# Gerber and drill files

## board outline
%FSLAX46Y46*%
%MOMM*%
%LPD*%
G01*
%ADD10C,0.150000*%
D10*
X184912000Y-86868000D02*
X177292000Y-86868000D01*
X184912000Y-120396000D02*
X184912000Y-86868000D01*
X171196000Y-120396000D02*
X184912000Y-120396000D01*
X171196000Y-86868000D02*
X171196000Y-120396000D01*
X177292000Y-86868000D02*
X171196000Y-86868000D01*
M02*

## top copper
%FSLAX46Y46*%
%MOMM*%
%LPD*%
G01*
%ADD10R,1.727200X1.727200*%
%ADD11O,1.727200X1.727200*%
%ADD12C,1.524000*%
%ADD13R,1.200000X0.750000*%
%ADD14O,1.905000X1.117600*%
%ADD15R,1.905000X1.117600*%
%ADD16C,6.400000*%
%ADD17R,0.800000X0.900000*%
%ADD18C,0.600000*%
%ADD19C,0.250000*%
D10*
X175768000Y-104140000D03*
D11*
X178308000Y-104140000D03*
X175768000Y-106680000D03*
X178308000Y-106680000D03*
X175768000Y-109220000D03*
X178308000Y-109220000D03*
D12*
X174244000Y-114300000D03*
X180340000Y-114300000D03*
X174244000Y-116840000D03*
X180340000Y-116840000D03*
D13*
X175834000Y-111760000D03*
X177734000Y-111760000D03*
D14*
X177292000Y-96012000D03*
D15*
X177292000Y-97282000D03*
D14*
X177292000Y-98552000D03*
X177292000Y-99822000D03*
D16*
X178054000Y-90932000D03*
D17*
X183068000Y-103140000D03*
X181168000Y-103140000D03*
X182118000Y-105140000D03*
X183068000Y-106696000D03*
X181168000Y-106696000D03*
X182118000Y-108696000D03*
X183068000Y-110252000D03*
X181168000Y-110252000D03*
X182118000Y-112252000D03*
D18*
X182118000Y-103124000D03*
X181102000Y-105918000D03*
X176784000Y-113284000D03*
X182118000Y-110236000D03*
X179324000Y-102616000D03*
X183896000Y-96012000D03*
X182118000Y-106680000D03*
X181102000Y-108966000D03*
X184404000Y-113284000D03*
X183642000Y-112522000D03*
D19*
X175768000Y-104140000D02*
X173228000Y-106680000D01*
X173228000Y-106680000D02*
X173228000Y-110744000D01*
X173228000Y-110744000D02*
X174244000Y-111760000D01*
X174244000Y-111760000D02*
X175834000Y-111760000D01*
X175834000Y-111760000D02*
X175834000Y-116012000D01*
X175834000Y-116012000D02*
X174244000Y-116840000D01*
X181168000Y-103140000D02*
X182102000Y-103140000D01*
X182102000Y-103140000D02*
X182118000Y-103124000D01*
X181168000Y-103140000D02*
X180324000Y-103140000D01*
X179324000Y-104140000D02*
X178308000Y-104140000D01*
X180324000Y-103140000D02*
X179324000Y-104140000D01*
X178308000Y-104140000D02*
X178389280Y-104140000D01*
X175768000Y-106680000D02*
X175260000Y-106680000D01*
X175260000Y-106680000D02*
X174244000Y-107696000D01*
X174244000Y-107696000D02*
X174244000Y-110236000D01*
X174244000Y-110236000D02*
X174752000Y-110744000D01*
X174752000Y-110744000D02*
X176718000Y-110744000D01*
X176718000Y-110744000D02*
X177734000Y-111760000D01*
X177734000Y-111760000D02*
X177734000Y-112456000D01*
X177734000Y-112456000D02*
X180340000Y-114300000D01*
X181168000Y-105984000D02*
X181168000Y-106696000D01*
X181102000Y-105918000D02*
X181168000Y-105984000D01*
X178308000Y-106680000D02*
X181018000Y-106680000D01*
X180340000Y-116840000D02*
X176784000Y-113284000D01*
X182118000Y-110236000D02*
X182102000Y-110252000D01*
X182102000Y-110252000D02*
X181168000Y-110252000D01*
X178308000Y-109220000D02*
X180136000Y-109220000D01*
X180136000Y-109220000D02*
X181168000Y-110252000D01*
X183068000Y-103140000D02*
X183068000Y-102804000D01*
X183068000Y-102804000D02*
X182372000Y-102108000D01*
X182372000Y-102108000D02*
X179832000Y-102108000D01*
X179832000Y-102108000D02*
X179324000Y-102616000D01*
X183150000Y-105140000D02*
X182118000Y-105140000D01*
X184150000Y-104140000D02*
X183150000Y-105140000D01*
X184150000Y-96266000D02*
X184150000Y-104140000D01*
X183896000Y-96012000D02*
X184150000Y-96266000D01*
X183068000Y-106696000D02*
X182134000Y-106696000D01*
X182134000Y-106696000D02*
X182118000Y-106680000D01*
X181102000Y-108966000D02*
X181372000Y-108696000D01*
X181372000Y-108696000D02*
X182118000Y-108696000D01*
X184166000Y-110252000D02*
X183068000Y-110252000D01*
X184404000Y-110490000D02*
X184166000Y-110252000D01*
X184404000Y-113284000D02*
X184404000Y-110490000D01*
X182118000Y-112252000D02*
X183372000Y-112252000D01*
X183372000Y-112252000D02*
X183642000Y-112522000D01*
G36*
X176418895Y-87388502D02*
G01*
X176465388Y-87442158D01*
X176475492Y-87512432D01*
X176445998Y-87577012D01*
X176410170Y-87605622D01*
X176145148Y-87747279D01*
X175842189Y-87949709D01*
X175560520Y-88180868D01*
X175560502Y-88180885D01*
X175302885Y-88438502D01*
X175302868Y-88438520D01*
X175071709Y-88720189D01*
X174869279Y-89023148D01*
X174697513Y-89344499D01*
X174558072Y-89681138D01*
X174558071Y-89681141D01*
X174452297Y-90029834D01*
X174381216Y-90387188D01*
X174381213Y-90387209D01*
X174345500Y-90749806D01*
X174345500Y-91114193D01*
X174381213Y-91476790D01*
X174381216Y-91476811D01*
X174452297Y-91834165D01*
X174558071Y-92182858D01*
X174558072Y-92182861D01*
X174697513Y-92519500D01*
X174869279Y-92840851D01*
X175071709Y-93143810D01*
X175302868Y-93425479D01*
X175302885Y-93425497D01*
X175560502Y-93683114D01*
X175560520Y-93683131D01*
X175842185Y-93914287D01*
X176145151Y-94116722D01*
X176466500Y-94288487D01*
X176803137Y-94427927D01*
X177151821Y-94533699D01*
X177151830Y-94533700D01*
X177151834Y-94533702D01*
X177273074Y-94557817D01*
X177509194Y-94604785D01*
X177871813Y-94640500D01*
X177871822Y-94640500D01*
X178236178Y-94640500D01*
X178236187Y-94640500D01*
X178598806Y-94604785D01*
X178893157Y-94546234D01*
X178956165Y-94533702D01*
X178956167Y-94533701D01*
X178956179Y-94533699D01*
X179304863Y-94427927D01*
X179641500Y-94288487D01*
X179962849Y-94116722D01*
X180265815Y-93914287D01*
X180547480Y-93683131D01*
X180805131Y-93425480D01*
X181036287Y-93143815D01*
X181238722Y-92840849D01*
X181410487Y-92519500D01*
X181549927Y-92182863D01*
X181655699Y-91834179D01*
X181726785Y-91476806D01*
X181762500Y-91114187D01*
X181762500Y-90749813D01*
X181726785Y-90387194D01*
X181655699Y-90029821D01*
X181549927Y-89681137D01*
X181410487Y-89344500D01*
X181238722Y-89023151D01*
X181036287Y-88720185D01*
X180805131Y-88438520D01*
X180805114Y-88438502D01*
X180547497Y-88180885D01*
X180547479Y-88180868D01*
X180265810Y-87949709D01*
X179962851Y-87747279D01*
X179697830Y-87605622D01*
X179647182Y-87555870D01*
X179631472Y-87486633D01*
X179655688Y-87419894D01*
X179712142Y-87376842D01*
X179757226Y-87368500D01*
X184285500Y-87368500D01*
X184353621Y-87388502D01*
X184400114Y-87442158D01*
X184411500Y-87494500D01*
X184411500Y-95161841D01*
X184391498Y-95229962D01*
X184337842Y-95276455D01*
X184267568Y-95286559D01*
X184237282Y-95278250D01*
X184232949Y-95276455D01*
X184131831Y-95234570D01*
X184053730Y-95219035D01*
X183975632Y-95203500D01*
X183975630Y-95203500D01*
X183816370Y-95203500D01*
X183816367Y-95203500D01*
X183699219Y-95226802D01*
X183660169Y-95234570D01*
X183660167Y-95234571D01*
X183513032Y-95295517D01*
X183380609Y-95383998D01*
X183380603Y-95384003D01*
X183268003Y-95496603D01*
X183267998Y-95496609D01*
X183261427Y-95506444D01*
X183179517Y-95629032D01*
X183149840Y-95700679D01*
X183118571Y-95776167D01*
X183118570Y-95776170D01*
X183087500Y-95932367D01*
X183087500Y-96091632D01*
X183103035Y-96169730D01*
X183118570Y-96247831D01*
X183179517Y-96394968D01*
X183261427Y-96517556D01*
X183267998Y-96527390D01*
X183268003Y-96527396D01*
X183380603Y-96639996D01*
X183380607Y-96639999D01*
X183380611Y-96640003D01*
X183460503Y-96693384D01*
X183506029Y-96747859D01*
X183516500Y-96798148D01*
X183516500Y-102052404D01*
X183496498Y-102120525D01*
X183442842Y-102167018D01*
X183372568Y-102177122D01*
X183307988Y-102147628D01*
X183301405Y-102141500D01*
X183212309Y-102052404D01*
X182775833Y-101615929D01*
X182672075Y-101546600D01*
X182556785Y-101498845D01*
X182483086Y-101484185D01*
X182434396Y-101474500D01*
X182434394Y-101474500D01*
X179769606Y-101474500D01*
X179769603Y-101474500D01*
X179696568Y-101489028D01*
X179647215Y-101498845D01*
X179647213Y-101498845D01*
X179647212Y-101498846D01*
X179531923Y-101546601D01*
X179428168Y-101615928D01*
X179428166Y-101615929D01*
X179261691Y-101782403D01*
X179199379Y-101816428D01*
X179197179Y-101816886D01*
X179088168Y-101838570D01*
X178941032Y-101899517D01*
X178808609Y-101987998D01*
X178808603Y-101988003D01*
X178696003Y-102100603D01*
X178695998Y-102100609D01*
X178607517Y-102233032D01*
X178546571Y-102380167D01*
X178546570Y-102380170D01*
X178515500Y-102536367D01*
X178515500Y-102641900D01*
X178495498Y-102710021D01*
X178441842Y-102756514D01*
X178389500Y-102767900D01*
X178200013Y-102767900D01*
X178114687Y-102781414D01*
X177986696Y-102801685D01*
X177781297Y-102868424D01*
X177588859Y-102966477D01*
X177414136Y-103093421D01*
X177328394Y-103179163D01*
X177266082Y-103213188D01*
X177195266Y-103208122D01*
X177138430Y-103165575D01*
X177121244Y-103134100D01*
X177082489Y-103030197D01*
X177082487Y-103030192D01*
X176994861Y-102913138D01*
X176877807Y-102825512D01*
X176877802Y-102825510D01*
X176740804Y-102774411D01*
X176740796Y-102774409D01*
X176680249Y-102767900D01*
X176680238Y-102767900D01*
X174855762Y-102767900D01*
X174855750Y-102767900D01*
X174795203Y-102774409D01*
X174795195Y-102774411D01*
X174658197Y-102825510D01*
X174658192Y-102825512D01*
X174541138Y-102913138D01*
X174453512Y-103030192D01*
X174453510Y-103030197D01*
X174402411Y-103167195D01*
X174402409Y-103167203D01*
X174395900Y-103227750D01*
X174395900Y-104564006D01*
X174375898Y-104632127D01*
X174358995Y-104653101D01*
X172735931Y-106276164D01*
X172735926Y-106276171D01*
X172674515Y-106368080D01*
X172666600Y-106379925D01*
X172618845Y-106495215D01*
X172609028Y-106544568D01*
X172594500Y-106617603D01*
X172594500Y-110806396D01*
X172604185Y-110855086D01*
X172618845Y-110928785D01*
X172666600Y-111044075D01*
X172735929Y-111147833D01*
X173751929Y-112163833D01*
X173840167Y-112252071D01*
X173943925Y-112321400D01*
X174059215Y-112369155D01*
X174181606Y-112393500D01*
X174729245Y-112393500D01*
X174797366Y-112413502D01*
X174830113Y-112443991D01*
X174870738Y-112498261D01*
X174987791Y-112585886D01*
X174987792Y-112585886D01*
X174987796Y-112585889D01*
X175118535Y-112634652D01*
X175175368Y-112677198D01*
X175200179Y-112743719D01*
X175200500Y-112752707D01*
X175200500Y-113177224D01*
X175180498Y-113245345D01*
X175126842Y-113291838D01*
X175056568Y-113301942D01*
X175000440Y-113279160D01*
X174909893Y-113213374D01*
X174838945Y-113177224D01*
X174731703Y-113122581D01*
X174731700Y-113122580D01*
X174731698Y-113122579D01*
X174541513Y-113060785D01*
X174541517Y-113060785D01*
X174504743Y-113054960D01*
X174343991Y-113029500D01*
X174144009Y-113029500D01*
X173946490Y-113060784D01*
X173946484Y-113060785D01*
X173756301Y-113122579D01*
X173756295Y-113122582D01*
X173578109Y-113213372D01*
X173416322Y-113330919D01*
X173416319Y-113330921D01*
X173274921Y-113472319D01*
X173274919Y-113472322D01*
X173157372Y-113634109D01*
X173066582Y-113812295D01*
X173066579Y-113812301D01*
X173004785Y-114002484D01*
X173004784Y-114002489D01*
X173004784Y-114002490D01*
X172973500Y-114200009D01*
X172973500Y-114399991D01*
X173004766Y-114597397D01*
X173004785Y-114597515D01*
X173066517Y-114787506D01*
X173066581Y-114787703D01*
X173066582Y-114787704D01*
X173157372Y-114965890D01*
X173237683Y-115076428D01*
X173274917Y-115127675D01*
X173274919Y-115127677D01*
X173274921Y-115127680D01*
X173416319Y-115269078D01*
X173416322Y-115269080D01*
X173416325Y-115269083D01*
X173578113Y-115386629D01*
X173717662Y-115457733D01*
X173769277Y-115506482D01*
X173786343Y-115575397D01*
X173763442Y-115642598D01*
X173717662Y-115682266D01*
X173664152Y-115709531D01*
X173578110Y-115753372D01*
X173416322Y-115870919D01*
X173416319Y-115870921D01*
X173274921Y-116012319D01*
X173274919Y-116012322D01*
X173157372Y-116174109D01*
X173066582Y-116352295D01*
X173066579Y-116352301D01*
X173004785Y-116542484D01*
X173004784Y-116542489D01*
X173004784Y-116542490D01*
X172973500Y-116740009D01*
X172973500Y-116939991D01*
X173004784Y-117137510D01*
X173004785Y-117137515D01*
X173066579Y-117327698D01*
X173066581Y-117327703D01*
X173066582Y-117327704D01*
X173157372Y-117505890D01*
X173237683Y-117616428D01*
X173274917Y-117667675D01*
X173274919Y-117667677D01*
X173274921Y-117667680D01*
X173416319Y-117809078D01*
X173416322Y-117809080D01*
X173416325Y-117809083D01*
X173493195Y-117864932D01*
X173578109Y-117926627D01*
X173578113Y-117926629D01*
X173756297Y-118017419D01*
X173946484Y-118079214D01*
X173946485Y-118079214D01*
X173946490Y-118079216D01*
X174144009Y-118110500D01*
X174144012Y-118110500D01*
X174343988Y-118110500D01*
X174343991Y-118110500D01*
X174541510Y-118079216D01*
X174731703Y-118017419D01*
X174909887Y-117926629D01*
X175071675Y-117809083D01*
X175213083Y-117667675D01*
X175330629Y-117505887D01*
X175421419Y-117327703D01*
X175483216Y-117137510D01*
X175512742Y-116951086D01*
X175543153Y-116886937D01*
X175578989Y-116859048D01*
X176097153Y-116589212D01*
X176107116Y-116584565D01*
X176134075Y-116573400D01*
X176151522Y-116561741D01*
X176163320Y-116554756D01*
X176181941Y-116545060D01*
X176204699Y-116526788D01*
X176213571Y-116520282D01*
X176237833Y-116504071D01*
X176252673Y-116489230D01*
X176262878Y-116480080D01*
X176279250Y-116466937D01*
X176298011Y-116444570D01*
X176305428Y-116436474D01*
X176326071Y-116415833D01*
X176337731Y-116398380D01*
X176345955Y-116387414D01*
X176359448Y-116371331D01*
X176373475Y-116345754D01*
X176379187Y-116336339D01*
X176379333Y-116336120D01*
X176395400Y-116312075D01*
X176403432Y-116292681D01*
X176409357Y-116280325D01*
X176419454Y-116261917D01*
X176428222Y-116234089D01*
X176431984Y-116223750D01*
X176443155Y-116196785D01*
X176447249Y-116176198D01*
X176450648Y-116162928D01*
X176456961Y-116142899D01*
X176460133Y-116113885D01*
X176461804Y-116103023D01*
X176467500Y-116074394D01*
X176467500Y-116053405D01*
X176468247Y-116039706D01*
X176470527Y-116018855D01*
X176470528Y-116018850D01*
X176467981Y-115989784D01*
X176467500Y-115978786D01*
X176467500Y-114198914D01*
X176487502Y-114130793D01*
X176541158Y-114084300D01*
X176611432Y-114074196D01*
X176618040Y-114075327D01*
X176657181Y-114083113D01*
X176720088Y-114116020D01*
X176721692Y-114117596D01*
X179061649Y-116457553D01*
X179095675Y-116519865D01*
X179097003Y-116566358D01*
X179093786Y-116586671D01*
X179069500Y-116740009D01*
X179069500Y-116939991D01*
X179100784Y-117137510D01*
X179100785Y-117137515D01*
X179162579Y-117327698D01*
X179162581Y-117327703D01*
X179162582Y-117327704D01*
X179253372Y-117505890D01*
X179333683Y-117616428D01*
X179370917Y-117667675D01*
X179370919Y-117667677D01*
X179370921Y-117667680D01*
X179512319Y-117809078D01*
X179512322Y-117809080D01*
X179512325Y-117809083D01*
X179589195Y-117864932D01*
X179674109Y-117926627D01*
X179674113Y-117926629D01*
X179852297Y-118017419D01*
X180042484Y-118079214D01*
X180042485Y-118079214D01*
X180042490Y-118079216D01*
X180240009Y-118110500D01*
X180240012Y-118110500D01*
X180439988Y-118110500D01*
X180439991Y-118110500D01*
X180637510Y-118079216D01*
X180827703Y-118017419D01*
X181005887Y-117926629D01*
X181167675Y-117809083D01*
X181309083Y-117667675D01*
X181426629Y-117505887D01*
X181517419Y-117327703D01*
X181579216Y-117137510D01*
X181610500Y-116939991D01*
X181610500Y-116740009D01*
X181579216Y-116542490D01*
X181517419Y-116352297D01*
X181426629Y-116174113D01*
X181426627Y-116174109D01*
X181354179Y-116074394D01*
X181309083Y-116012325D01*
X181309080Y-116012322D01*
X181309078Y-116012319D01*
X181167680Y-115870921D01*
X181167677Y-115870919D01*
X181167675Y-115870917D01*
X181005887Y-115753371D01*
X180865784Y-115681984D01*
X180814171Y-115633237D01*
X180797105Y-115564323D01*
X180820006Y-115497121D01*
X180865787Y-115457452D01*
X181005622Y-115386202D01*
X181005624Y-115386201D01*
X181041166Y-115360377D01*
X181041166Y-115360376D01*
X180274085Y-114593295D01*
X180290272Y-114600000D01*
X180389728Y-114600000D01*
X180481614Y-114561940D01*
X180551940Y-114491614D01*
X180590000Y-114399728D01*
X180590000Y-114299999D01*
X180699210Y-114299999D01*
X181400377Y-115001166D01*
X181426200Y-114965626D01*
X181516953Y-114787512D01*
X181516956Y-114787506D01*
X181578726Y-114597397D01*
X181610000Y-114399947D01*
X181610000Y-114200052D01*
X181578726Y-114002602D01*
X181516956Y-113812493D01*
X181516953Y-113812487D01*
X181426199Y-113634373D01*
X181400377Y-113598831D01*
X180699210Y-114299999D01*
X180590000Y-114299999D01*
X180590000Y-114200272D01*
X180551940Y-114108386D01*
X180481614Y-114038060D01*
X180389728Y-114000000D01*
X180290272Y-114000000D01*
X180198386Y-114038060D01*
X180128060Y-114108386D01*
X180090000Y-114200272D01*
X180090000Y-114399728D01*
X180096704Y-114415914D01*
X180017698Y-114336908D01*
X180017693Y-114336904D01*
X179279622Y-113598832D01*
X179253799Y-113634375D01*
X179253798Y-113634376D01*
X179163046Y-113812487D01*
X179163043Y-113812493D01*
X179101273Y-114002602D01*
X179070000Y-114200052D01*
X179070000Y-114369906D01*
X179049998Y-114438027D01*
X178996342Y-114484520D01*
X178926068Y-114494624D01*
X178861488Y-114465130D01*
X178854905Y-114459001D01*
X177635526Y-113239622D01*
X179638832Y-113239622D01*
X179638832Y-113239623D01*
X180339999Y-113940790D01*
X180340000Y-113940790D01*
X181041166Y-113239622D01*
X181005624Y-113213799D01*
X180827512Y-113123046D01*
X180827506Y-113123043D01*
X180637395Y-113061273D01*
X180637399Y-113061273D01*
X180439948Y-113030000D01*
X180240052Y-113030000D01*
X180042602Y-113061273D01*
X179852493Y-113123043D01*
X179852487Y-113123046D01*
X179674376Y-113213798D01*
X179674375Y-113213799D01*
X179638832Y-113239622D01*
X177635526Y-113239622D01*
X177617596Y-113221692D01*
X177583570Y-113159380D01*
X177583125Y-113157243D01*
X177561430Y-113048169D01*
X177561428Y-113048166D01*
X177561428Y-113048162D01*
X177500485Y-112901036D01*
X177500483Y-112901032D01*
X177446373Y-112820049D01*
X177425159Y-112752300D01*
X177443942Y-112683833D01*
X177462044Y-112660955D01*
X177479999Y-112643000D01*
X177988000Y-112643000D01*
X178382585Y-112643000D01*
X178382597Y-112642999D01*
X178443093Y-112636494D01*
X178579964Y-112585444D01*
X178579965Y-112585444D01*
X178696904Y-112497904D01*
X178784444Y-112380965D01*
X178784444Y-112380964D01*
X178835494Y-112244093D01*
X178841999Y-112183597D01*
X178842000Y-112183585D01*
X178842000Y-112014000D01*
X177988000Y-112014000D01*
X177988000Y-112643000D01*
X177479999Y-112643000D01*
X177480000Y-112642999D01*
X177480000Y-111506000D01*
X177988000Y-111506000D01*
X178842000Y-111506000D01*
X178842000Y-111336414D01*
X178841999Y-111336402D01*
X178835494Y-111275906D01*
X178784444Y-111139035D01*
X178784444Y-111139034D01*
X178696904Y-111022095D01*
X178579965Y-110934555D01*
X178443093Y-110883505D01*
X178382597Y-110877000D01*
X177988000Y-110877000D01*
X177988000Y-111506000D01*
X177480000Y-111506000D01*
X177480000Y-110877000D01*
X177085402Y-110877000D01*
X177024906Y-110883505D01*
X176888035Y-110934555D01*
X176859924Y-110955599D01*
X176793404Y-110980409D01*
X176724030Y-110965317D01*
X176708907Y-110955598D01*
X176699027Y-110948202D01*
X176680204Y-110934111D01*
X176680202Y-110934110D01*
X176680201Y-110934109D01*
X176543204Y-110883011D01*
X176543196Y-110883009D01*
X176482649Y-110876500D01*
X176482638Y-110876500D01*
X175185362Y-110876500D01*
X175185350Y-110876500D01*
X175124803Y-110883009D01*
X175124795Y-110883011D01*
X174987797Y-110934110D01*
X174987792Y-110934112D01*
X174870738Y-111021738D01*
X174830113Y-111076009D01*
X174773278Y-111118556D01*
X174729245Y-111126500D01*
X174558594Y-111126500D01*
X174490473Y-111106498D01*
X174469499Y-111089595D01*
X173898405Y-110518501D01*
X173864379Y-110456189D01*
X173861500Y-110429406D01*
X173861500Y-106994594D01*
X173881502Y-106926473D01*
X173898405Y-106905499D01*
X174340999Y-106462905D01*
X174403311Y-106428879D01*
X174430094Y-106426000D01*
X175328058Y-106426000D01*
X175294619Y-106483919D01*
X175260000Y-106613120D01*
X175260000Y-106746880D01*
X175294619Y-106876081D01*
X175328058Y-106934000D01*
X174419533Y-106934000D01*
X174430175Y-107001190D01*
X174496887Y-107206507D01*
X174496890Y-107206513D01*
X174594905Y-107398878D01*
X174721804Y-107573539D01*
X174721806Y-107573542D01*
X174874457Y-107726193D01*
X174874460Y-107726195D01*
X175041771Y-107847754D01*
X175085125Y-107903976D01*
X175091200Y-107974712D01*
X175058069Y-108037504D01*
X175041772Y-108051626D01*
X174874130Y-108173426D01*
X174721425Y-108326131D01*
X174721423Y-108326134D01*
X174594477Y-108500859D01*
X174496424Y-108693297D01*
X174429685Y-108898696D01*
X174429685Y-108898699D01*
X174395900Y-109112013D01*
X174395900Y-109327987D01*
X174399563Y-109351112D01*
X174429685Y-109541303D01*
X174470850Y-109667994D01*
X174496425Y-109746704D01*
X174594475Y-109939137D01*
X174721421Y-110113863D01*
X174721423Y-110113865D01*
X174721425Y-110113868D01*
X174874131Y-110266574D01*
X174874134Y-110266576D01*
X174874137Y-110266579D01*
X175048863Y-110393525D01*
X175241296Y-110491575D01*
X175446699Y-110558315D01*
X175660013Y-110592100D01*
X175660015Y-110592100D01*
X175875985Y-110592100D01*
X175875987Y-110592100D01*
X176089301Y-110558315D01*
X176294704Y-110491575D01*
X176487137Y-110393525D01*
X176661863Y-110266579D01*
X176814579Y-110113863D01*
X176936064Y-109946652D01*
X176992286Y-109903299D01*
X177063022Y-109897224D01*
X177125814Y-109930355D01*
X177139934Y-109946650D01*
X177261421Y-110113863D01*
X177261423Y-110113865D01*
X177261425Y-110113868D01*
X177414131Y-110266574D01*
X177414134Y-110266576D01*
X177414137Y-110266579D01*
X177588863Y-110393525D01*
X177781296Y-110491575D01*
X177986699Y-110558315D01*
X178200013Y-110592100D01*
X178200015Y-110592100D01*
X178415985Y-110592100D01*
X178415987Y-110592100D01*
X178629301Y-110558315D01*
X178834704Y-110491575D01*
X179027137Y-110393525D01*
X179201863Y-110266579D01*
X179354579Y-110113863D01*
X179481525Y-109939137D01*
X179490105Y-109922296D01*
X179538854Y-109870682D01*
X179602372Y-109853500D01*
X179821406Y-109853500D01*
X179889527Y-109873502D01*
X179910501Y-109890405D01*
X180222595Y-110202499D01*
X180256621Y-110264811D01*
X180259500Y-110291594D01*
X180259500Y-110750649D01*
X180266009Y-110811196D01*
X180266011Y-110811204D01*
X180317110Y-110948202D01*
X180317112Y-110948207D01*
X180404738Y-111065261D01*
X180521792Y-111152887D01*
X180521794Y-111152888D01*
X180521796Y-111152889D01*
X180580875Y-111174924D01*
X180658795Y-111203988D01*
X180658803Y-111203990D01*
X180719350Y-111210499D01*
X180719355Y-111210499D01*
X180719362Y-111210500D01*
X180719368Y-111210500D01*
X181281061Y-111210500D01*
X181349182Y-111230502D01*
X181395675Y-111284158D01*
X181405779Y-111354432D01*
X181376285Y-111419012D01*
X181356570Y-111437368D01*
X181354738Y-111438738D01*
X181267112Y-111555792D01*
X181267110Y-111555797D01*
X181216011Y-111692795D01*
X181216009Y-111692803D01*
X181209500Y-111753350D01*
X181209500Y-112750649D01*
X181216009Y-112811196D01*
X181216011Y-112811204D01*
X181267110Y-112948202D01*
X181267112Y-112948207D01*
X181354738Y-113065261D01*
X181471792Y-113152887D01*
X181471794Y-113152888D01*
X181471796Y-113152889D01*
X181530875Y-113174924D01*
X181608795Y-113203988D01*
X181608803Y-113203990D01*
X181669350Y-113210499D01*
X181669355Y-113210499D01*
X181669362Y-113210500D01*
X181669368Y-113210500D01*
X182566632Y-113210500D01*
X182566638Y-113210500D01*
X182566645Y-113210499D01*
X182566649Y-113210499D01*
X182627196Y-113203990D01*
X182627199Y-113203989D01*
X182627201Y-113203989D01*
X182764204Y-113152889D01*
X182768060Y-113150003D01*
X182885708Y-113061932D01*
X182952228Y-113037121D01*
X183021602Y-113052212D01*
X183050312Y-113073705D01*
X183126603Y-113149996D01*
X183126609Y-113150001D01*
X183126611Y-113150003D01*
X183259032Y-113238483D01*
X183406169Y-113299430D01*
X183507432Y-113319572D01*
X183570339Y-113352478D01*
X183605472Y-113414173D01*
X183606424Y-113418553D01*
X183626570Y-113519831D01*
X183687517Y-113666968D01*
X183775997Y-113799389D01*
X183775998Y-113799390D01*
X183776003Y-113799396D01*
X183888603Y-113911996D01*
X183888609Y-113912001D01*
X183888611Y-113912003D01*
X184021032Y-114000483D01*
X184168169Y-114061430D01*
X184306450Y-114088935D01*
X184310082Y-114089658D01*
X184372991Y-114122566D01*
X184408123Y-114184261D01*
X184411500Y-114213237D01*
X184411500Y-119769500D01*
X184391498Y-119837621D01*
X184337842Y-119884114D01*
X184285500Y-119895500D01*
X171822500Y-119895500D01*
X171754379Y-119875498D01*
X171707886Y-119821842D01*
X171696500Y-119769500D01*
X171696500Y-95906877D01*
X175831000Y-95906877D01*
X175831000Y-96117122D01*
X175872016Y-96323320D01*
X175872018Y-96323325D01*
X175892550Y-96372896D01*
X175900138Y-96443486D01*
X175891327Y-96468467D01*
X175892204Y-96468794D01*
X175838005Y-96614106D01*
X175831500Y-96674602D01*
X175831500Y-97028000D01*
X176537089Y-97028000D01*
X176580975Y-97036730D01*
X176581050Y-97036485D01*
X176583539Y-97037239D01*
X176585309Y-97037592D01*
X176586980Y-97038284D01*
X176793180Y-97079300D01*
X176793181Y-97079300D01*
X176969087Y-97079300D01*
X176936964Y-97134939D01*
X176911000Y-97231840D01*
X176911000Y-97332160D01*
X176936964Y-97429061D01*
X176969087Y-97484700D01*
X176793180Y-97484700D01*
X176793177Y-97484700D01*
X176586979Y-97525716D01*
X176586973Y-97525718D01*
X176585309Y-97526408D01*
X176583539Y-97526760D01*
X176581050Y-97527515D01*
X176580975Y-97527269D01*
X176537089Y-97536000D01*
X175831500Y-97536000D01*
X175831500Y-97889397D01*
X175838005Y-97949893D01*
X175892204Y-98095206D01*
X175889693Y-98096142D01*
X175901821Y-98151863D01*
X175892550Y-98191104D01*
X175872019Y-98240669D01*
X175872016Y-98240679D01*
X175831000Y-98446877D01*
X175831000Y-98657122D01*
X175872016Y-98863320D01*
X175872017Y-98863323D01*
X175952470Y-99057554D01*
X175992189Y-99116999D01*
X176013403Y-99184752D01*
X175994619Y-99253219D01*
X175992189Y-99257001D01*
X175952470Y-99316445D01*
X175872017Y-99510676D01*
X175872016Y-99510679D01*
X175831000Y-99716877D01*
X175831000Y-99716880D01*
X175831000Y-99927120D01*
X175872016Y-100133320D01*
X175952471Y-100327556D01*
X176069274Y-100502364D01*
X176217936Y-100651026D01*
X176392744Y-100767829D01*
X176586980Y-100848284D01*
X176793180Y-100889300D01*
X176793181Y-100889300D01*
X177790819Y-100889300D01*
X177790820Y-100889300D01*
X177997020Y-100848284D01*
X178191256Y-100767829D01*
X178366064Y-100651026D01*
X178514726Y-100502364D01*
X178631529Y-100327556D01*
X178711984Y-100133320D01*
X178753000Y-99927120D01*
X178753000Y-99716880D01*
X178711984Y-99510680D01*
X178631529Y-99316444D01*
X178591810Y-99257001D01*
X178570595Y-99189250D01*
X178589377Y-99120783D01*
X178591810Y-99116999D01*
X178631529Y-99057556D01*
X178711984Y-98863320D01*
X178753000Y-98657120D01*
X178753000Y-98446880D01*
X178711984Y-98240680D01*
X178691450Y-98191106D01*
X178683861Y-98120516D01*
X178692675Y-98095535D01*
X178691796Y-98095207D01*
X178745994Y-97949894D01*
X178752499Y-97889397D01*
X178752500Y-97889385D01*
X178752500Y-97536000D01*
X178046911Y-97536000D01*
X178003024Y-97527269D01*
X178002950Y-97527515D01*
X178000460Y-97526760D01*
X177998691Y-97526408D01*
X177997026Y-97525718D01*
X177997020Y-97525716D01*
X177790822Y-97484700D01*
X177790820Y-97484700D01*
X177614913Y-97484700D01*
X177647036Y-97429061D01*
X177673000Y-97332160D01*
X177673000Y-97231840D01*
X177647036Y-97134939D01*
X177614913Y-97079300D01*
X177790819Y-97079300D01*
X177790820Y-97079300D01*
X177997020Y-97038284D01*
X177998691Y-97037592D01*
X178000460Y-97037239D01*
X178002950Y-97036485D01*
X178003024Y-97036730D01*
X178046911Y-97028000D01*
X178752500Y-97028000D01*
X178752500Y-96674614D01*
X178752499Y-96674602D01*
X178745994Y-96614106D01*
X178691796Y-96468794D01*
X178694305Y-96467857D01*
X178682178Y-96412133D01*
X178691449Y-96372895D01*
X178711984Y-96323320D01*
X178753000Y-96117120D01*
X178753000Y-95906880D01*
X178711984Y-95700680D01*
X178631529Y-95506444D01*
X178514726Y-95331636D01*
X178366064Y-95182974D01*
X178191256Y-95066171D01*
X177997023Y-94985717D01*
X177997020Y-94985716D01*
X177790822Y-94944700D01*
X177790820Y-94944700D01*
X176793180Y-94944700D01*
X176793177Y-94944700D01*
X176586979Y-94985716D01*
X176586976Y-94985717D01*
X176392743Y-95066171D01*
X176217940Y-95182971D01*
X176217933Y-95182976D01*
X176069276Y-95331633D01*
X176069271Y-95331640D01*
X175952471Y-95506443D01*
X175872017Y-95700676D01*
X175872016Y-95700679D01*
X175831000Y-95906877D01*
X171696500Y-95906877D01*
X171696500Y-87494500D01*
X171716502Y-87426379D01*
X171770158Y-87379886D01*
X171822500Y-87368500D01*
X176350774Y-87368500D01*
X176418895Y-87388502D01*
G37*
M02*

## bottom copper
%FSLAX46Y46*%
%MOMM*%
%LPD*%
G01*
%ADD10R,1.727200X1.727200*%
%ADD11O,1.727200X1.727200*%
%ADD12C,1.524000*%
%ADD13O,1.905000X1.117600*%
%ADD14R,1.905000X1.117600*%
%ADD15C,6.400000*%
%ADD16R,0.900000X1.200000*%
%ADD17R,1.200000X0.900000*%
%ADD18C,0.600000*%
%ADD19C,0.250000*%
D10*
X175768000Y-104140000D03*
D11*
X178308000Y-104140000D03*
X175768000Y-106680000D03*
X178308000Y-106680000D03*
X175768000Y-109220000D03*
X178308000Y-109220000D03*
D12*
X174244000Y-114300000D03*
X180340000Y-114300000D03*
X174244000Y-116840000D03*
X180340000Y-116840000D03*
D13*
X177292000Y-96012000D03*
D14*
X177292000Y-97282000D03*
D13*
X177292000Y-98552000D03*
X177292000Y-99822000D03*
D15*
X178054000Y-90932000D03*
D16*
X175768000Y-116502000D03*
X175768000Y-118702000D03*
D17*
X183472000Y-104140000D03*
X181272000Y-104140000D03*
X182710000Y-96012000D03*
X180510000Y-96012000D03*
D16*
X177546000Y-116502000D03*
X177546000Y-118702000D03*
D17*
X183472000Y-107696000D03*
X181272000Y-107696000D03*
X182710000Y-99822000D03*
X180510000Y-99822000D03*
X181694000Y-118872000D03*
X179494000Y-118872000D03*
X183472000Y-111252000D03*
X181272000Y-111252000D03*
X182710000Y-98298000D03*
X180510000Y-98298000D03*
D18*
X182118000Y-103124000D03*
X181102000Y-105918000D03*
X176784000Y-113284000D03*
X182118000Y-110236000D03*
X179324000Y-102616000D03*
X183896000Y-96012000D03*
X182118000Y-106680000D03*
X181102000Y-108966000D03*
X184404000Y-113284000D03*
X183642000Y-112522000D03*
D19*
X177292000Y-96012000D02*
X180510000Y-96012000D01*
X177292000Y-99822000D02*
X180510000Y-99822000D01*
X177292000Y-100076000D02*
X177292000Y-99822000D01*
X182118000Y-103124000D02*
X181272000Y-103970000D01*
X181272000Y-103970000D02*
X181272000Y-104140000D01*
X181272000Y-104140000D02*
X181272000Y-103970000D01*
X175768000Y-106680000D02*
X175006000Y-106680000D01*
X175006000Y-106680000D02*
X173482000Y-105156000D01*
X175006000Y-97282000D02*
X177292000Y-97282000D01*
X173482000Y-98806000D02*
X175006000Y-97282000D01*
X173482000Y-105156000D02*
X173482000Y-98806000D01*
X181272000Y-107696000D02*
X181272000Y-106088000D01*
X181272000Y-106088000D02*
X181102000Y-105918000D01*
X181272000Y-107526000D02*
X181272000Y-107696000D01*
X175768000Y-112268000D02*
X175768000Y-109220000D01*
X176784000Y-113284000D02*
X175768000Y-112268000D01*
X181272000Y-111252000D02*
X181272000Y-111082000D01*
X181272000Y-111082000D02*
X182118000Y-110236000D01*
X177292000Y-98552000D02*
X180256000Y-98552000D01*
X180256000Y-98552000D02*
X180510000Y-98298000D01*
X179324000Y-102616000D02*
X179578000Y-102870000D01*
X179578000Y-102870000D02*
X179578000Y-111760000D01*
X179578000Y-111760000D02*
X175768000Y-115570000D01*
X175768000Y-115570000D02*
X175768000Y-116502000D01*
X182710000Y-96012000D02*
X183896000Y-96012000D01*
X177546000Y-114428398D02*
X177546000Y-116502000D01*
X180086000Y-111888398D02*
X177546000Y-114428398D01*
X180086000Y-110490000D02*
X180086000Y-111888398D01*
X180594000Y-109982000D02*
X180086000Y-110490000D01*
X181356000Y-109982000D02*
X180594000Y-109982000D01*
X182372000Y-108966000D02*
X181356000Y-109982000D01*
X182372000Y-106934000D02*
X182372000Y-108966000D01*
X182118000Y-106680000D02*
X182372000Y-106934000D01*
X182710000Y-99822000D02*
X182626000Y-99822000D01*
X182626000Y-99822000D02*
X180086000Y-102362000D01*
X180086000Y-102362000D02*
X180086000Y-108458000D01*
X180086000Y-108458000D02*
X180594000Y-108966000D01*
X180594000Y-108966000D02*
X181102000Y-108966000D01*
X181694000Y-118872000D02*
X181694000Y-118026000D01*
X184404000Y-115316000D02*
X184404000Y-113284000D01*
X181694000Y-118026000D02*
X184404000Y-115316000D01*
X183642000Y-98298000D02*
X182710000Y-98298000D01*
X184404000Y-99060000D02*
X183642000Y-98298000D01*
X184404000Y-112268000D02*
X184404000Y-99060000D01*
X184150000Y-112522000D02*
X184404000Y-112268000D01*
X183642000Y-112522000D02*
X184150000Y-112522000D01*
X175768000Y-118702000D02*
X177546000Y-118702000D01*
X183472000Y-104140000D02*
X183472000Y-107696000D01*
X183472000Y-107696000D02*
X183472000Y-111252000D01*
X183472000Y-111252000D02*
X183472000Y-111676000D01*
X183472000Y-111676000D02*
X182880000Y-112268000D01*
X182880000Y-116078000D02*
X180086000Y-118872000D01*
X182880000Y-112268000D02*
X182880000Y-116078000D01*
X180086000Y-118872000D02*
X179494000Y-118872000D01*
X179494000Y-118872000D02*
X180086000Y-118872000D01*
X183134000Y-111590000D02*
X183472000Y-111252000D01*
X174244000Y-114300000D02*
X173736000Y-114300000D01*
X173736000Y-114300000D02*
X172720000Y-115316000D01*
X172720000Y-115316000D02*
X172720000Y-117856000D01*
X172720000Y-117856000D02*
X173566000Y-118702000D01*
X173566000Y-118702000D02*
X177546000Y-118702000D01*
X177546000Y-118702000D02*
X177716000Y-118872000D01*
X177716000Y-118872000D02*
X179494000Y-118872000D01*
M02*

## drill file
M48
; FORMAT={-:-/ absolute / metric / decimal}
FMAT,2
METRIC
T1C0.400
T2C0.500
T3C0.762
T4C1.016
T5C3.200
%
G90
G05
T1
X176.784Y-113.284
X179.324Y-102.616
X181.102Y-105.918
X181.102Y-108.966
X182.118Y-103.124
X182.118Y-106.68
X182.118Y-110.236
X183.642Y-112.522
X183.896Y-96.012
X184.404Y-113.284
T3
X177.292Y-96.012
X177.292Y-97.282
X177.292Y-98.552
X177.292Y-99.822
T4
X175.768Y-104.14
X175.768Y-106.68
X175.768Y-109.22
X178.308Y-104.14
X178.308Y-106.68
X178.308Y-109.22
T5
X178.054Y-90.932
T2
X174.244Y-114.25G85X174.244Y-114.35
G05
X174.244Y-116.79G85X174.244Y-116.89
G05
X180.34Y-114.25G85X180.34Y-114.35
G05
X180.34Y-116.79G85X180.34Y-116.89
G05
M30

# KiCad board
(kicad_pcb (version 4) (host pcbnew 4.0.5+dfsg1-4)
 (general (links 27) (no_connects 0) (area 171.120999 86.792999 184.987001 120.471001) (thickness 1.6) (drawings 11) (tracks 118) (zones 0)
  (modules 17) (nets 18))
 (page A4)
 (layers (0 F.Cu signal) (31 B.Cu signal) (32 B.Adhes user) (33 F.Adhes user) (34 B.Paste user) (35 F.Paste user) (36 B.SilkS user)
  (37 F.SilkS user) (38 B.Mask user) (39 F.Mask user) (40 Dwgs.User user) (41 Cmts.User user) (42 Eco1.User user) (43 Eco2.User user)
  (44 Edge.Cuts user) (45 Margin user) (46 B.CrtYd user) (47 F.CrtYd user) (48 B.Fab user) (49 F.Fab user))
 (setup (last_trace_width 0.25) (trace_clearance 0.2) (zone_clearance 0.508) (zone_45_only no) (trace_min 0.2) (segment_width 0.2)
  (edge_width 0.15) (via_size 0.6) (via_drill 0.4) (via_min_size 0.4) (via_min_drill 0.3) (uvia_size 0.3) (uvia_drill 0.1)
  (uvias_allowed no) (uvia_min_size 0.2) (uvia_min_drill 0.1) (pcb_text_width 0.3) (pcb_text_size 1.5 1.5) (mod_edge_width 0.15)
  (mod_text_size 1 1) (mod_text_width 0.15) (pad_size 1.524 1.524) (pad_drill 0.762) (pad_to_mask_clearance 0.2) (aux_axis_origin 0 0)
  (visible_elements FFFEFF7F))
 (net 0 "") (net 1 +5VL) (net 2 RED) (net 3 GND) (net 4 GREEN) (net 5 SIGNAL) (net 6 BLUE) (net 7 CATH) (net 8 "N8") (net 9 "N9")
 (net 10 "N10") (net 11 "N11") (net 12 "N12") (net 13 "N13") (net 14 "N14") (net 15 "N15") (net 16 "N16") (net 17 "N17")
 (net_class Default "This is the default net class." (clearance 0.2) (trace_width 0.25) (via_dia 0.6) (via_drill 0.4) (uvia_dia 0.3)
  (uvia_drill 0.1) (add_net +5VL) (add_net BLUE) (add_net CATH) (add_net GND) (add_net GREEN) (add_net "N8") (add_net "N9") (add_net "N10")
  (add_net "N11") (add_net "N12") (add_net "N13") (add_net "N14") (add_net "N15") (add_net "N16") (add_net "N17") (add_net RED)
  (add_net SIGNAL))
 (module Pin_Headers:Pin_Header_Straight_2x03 (layer F.Cu) (at 175.768 104.14)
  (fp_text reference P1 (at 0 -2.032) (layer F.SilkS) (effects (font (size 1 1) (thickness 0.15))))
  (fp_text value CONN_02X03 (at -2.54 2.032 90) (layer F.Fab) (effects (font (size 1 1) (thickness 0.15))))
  (pad 1 thru_hole rect (at 0 0) (size 1.7272 1.7272) (drill 1.016) (layers *.Cu *.Mask) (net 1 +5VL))
  (pad 2 thru_hole oval (at 2.54 0) (size 1.7272 1.7272) (drill 1.016) (layers *.Cu *.Mask) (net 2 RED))
  (pad 3 thru_hole oval (at 0 2.54) (size 1.7272 1.7272) (drill 1.016) (layers *.Cu *.Mask) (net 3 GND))
  (pad 4 thru_hole oval (at 2.54 2.54) (size 1.7272 1.7272) (drill 1.016) (layers *.Cu *.Mask) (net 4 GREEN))
  (pad 5 thru_hole oval (at 0 5.08) (size 1.7272 1.7272) (drill 1.016) (layers *.Cu *.Mask) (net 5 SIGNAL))
  (pad 6 thru_hole oval (at 2.54 5.08) (size 1.7272 1.7272) (drill 1.016) (layers *.Cu *.Mask) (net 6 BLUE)))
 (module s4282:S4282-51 (layer F.Cu) (at 177.292 115.57)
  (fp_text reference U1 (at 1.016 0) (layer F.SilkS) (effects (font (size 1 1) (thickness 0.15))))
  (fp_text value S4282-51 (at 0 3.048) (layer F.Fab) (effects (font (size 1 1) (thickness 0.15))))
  (pad 1 thru_hole circle (at -3.048 -1.27) (size 1.524 1.524) (drill oval 0.5 0.6) (layers *.Cu *.Mask F.SilkS) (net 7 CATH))
  (pad 4 thru_hole circle (at 3.048 -1.27) (size 1.524 1.524) (drill oval 0.5 0.6) (layers *.Cu *.Mask F.SilkS) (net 3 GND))
  (pad 2 thru_hole circle (at -3.048 1.27) (size 1.524 1.524) (drill oval 0.5 0.6) (layers *.Cu *.Mask F.SilkS) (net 1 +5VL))
  (pad 3 thru_hole circle (at 3.048 1.27) (size 1.524 1.524) (drill oval 0.5 0.6) (layers *.Cu *.Mask F.SilkS) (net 5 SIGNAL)))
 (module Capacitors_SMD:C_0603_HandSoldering (layer F.Cu) (at 176.784 111.76)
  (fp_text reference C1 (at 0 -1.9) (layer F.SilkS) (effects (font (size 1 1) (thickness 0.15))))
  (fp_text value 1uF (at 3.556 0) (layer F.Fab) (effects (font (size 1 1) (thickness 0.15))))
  (pad 1 smd rect (at -0.95 0) (size 1.2 0.75) (layers F.Cu F.Paste F.Mask) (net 1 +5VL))
  (pad 2 smd rect (at 0.95 0) (size 1.2 0.75) (layers F.Cu F.Paste F.Mask) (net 3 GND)))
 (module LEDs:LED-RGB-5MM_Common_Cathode (layer F.Cu) (at 177.292 96.012)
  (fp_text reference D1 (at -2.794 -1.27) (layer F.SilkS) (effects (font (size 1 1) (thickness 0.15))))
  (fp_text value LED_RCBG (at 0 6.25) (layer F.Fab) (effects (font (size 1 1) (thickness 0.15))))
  (pad 1 thru_hole oval (at 0 0) (size 1.905 1.1176) (drill 0.762) (layers *.Cu *.Mask) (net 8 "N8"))
  (pad 2 thru_hole rect (at 0 1.27) (size 1.905 1.1176) (drill 0.762) (layers *.Cu *.Mask) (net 3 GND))
  (pad 3 thru_hole oval (at 0 2.54) (size 1.905 1.1176) (drill 0.762) (layers *.Cu *.Mask) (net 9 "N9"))
  (pad 4 thru_hole oval (at 0 3.81) (size 1.905 1.1176) (drill 0.762) (layers *.Cu *.Mask) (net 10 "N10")))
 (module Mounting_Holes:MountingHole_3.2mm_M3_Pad (layer F.Cu) (at 178.054 90.932)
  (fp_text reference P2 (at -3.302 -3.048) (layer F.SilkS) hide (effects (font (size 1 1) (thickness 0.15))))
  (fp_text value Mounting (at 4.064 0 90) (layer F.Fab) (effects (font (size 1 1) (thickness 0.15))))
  (pad 1 thru_hole circle (at 0 0) (size 6.4 6.4) (drill 3.2) (layers *.Cu *.Mask) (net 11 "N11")))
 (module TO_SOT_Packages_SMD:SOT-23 (layer F.Cu) (at 182.118 104.14 270)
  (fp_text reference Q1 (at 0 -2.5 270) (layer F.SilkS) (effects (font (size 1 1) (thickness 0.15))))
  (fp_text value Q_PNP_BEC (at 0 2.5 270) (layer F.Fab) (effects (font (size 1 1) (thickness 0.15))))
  (pad 1 smd rect (at -1 -0.95 270) (size 0.9 0.8) (layers F.Cu F.Paste F.Mask) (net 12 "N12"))
  (pad 2 smd rect (at -1 0.95 270) (size 0.9 0.8) (layers F.Cu F.Paste F.Mask) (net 2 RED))
  (pad 3 smd rect (at 1 0 270) (size 0.9 0.8) (layers F.Cu F.Paste F.Mask) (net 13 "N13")))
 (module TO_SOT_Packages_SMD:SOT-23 (layer F.Cu) (at 182.118 107.696 270)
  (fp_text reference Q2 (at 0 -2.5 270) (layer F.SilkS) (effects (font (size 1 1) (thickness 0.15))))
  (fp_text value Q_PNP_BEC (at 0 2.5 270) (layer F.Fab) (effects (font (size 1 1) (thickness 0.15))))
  (pad 1 smd rect (at -1 -0.95 270) (size 0.9 0.8) (layers F.Cu F.Paste F.Mask) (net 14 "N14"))
  (pad 2 smd rect (at -1 0.95 270) (size 0.9 0.8) (layers F.Cu F.Paste F.Mask) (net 4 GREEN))
  (pad 3 smd rect (at 1 0 270) (size 0.9 0.8) (layers F.Cu F.Paste F.Mask) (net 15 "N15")))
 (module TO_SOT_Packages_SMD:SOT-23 (layer F.Cu) (at 182.118 111.252 270)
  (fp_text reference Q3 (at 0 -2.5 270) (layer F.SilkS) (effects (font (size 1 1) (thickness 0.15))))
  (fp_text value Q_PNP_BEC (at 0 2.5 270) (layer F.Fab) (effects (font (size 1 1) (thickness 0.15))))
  (pad 1 smd rect (at -1 -0.95 270) (size 0.9 0.8) (layers F.Cu F.Paste F.Mask) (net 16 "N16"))
  (pad 2 smd rect (at -1 0.95 270) (size 0.9 0.8) (layers F.Cu F.Paste F.Mask) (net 6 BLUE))
  (pad 3 smd rect (at 1 0 270) (size 0.9 0.8) (layers F.Cu F.Paste F.Mask) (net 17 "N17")))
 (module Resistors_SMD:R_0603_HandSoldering (layer B.Cu) (at 175.768 117.602 270)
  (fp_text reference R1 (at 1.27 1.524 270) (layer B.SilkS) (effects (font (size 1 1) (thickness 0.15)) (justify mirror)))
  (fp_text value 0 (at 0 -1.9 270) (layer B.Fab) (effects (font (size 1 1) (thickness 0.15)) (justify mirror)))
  (pad 1 smd rect (at -1.1 0 270) (size 1.2 0.9) (layers B.Cu B.Paste B.Mask) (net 12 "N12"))
  (pad 2 smd rect (at 1.1 0 270) (size 1.2 0.9) (layers B.Cu B.Paste B.Mask) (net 7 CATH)))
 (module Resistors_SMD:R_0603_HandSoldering (layer B.Cu) (at 182.372 104.14 180)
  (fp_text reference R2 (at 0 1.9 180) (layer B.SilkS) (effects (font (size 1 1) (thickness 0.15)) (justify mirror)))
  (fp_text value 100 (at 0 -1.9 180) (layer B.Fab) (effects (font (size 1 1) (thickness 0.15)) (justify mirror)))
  (pad 1 smd rect (at -1.1 0 180) (size 1.2 0.9) (layers B.Cu B.Paste B.Mask) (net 7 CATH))
  (pad 2 smd rect (at 1.1 0 180) (size 1.2 0.9) (layers B.Cu B.Paste B.Mask) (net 2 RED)))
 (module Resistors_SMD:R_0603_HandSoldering (layer B.Cu) (at 181.61 96.012 180)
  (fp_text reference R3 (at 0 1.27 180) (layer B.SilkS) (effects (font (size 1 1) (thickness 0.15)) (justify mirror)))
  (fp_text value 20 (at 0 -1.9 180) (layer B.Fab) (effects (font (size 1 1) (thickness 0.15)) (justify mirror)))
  (pad 1 smd rect (at -1.1 0 180) (size 1.2 0.9) (layers B.Cu B.Paste B.Mask) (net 13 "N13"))
  (pad 2 smd rect (at 1.1 0 180) (size 1.2 0.9) (layers B.Cu B.Paste B.Mask) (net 8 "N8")))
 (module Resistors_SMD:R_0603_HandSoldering (layer B.Cu) (at 177.546 117.602 270)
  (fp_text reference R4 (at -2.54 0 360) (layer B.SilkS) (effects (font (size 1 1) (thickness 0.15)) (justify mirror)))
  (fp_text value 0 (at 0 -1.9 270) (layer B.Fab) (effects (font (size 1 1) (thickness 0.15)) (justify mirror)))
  (pad 1 smd rect (at -1.1 0 270) (size 1.2 0.9) (layers B.Cu B.Paste B.Mask) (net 14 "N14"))
  (pad 2 smd rect (at 1.1 0 270) (size 1.2 0.9) (layers B.Cu B.Paste B.Mask) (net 7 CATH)))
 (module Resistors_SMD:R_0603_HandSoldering (layer B.Cu) (at 182.372 107.696 180)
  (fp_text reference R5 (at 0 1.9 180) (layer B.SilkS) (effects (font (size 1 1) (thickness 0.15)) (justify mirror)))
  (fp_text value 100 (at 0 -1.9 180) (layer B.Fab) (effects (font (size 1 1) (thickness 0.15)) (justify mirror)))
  (pad 1 smd rect (at -1.1 0 180) (size 1.2 0.9) (layers B.Cu B.Paste B.Mask) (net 7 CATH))
  (pad 2 smd rect (at 1.1 0 180) (size 1.2 0.9) (layers B.Cu B.Paste B.Mask) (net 4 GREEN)))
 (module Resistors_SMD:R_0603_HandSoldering (layer B.Cu) (at 181.61 99.822 180)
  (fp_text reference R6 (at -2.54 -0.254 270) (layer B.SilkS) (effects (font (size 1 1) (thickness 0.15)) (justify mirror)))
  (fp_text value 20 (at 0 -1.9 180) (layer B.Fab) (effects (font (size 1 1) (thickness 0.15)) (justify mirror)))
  (pad 1 smd rect (at -1.1 0 180) (size 1.2 0.9) (layers B.Cu B.Paste B.Mask) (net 15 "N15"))
  (pad 2 smd rect (at 1.1 0 180) (size 1.2 0.9) (layers B.Cu B.Paste B.Mask) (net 10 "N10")))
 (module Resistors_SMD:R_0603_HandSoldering (layer B.Cu) (at 180.594 118.872 180)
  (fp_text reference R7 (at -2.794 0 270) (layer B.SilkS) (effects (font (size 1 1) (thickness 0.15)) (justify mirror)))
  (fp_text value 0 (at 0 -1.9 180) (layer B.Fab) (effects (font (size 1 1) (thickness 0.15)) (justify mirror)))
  (pad 1 smd rect (at -1.1 0 180) (size 1.2 0.9) (layers B.Cu B.Paste B.Mask) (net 16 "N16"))
  (pad 2 smd rect (at 1.1 0 180) (size 1.2 0.9) (layers B.Cu B.Paste B.Mask) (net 7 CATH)))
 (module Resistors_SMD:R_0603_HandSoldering (layer B.Cu) (at 182.372 111.252 180)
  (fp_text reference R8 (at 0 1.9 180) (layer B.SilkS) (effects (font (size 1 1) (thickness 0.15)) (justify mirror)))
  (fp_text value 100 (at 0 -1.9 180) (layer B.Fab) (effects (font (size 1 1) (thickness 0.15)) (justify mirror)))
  (pad 1 smd rect (at -1.1 0 180) (size 1.2 0.9) (layers B.Cu B.Paste B.Mask) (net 7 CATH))
  (pad 2 smd rect (at 1.1 0 180) (size 1.2 0.9) (layers B.Cu B.Paste B.Mask) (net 6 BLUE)))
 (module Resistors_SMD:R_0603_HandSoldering (layer B.Cu) (at 181.61 98.298 180)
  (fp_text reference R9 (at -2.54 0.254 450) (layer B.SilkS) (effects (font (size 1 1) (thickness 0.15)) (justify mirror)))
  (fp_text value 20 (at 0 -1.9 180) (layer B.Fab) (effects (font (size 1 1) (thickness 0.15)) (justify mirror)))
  (pad 1 smd rect (at -1.1 0 180) (size 1.2 0.9) (layers B.Cu B.Paste B.Mask) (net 17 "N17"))
  (pad 2 smd rect (at 1.1 0 180) (size 1.2 0.9) (layers B.Cu B.Paste B.Mask) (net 9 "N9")))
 (gr_line (start 184.912 86.868) (end 177.292 86.868) (angle 90) (layer Edge.Cuts) (width 0.15))
 (gr_line (start 184.912 120.396) (end 184.912 86.868) (angle 90) (layer Edge.Cuts) (width 0.15))
 (gr_line (start 171.196 120.396) (end 184.912 120.396) (angle 90) (layer Edge.Cuts) (width 0.15))
 (gr_line (start 171.196 86.868) (end 171.196 120.396) (angle 90) (layer Edge.Cuts) (width 0.15))
 (gr_line (start 177.292 86.868) (end 171.196 86.868) (angle 90) (layer Edge.Cuts) (width 0.15))
 (segment (start 177.292 96.012) (end 180.51 96.012) (width 0.25) (layer B.Cu) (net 8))
 (segment (start 177.292 99.822) (end 180.51 99.822) (width 0.25) (layer B.Cu) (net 10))
 (segment (start 177.292 100.076) (end 177.292 99.822) (width 0.25) (layer B.Cu) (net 10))
 (segment (start 175.768 104.14) (end 173.228 106.68) (width 0.25) (layer F.Cu) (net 1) (status 10))
 (segment (start 173.228 106.68) (end 173.228 110.744) (width 0.25) (layer F.Cu) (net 1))
 (segment (start 173.228 110.744) (end 174.244 111.76) (width 0.25) (layer F.Cu) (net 1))
 (segment (start 174.244 111.76) (end 175.834 111.76) (width 0.25) (layer F.Cu) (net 1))
 (segment (start 175.834 111.76) (end 175.834 116.012) (width 0.25) (layer F.Cu) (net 1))
 (segment (start 175.834 116.012) (end 174.244 116.84) (width 0.25) (layer F.Cu) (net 1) (status 20))
 (segment (start 181.168 103.14) (end 182.102 103.14) (width 0.25) (layer F.Cu) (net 2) (status 400000))
 (segment (start 182.118 103.124) (end 181.272 103.97) (width 0.25) (layer B.Cu) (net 2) (status 800000))
 (via (at 182.118 103.124) (size 0.6) (drill 0.4) (layers F.Cu B.Cu) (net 2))
 (segment (start 182.102 103.14) (end 182.118 103.124) (width 0.25) (layer F.Cu) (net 2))
 (segment (start 181.272 103.97) (end 181.272 104.14) (width 0.25) (layer B.Cu) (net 2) (status C00000))
 (segment (start 181.168 103.14) (end 180.324 103.14) (width 0.25) (layer F.Cu) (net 2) (status 400000))
 (segment (start 179.324 104.14) (end 178.308 104.14) (width 0.25) (layer F.Cu) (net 2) (status 800000))
 (segment (start 180.324 103.14) (end 179.324 104.14) (width 0.25) (layer F.Cu) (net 2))
 (segment (start 181.272 104.14) (end 181.272 103.97) (width 0.25) (layer B.Cu) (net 2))
 (segment (start 178.308 104.14) (end 178.38928 104.14) (width 0.25) (layer F.Cu) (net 2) (status 30))
 (segment (start 175.768 106.68) (end 175.006 106.68) (width 0.25) (layer B.Cu) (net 3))
 (segment (start 175.006 106.68) (end 173.482 105.156) (width 0.25) (layer B.Cu) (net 3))
 (segment (start 175.006 97.282) (end 177.292 97.282) (width 0.25) (layer B.Cu) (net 3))
 (segment (start 173.482 98.806) (end 175.006 97.282) (width 0.25) (layer B.Cu) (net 3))
 (segment (start 173.482 105.156) (end 173.482 98.806) (width 0.25) (layer B.Cu) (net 3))
 (segment (start 175.768 106.68) (end 175.26 106.68) (width 0.25) (layer F.Cu) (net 3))
 (segment (start 175.26 106.68) (end 174.244 107.696) (width 0.25) (layer F.Cu) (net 3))
 (segment (start 174.244 107.696) (end 174.244 110.236) (width 0.25) (layer F.Cu) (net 3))
 (segment (start 174.244 110.236) (end 174.752 110.744) (width 0.25) (layer F.Cu) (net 3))
 (segment (start 174.752 110.744) (end 176.718 110.744) (width 0.25) (layer F.Cu) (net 3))
 (segment (start 176.718 110.744) (end 177.734 111.76) (width 0.25) (layer F.Cu) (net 3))
 (segment (start 177.734 111.76) (end 177.734 112.456) (width 0.25) (layer F.Cu) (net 3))
 (segment (start 177.734 112.456) (end 180.34 114.3) (width 0.25) (layer F.Cu) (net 3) (status 20))
 (segment (start 181.272 107.696) (end 181.272 106.088) (width 0.25) (layer B.Cu) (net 4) (status 400000))
 (segment (start 181.168 105.984) (end 181.168 106.696) (width 0.25) (layer F.Cu) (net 4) (status 800000))
 (segment (start 181.102 105.918) (end 181.168 105.984) (width 0.25) (layer F.Cu) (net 4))
 (via (at 181.102 105.918) (size 0.6) (drill 0.4) (layers F.Cu B.Cu) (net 4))
 (segment (start 181.272 106.088) (end 181.102 105.918) (width 0.25) (layer B.Cu) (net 4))
 (segment (start 181.272 107.526) (end 181.272 107.696) (width 0.25) (layer B.Cu) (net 4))
 (segment (start 178.308 106.68) (end 181.018 106.68) (width 0.25) (layer F.Cu) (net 4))
 (segment (start 180.34 116.84) (end 176.784 113.284) (width 0.25) (layer F.Cu) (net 5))
 (segment (start 175.768 112.268) (end 175.768 109.22) (width 0.25) (layer B.Cu) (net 5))
 (segment (start 176.784 113.284) (end 175.768 112.268) (width 0.25) (layer B.Cu) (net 5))
 (via (at 176.784 113.284) (size 0.6) (drill 0.4) (layers F.Cu B.Cu) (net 5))
 (segment (start 181.272 111.252) (end 181.272 111.082) (width 0.25) (layer B.Cu) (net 6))
 (segment (start 181.272 111.082) (end 182.118 110.236) (width 0.25) (layer B.Cu) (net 6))
 (via (at 182.118 110.236) (size 0.6) (drill 0.4) (layers F.Cu B.Cu) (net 6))
 (segment (start 182.118 110.236) (end 182.102 110.252) (width 0.25) (layer F.Cu) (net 6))
 (segment (start 182.102 110.252) (end 181.168 110.252) (width 0.25) (layer F.Cu) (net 6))
 (segment (start 178.308 109.22) (end 180.136 109.22) (width 0.25) (layer F.Cu) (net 6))
 (segment (start 180.136 109.22) (end 181.168 110.252) (width 0.25) (layer F.Cu) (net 6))
 (segment (start 177.292 98.552) (end 180.256 98.552) (width 0.25) (layer B.Cu) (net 9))
 (segment (start 180.256 98.552) (end 180.51 98.298) (width 0.25) (layer B.Cu) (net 9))
 (segment (start 183.068 103.14) (end 183.068 102.804) (width 0.25) (layer F.Cu) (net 12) (status C00000))
 (segment (start 183.068 102.804) (end 182.372 102.108) (width 0.25) (layer F.Cu) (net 12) (status 400000))
 (segment (start 182.372 102.108) (end 179.832 102.108) (width 0.25) (layer F.Cu) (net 12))
 (segment (start 179.832 102.108) (end 179.324 102.616) (width 0.25) (layer F.Cu) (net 12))
 (via (at 179.324 102.616) (size 0.6) (drill 0.4) (layers F.Cu B.Cu) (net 12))
 (segment (start 179.324 102.616) (end 179.578 102.87) (width 0.25) (layer B.Cu) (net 12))
 (segment (start 179.578 102.87) (end 179.578 111.76) (width 0.25) (layer B.Cu) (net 12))
 (segment (start 179.578 111.76) (end 175.768 115.57) (width 0.25) (layer B.Cu) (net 12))
 (segment (start 175.768 115.57) (end 175.768 116.502) (width 0.25) (layer B.Cu) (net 12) (status 800000))
 (segment (start 182.71 96.012) (end 183.896 96.012) (width 0.25) (layer B.Cu) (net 13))
 (segment (start 183.15 105.14) (end 182.118 105.14) (width 0.25) (layer F.Cu) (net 13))
 (segment (start 184.15 104.14) (end 183.15 105.14) (width 0.25) (layer F.Cu) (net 13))
 (segment (start 184.15 96.266) (end 184.15 104.14) (width 0.25) (layer F.Cu) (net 13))
 (segment (start 183.896 96.012) (end 184.15 96.266) (width 0.25) (layer F.Cu) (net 13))
 (via (at 183.896 96.012) (size 0.6) (drill 0.4) (layers F.Cu B.Cu) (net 13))
 (segment (start 183.068 106.696) (end 182.134 106.696) (width 0.25) (layer F.Cu) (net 14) (status 400000))
 (segment (start 177.546 114.428398) (end 177.546 116.502) (width 0.25) (layer B.Cu) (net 14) (status 800000))
 (segment (start 180.086 111.888398) (end 177.546 114.428398) (width 0.25) (layer B.Cu) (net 14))
 (segment (start 180.086 110.49) (end 180.086 111.888398) (width 0.25) (layer B.Cu) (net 14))
 (segment (start 180.594 109.982) (end 180.086 110.49) (width 0.25) (layer B.Cu) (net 14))
 (segment (start 181.356 109.982) (end 180.594 109.982) (width 0.25) (layer B.Cu) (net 14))
 (segment (start 182.372 108.966) (end 181.356 109.982) (width 0.25) (layer B.Cu) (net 14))
 (segment (start 182.372 106.934) (end 182.372 108.966) (width 0.25) (layer B.Cu) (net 14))
 (segment (start 182.118 106.68) (end 182.372 106.934) (width 0.25) (layer B.Cu) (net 14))
 (via (at 182.118 106.68) (size 0.6) (drill 0.4) (layers F.Cu B.Cu) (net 14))
 (segment (start 182.134 106.696) (end 182.118 106.68) (width 0.25) (layer F.Cu) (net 14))
 (segment (start 182.71 99.822) (end 182.626 99.822) (width 0.25) (layer B.Cu) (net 15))
 (segment (start 182.626 99.822) (end 180.086 102.362) (width 0.25) (layer B.Cu) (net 15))
 (segment (start 180.086 102.362) (end 180.086 108.458) (width 0.25) (layer B.Cu) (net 15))
 (segment (start 180.086 108.458) (end 180.594 108.966) (width 0.25) (layer B.Cu) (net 15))
 (segment (start 180.594 108.966) (end 181.102 108.966) (width 0.25) (layer B.Cu) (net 15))
 (via (at 181.102 108.966) (size 0.6) (drill 0.4) (layers F.Cu B.Cu) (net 15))
 (segment (start 181.102 108.966) (end 181.372 108.696) (width 0.25) (layer F.Cu) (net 15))
 (segment (start 181.372 108.696) (end 182.118 108.696) (width 0.25) (layer F.Cu) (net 15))
 (segment (start 181.694 118.872) (end 181.694 118.026) (width 0.25) (layer B.Cu) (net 16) (status 400000))
 (segment (start 184.166 110.252) (end 183.068 110.252) (width 0.25) (layer F.Cu) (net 16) (status 800000))
 (segment (start 184.404 110.49) (end 184.166 110.252) (width 0.25) (layer F.Cu) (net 16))
 (segment (start 184.404 113.284) (end 184.404 110.49) (width 0.25) (layer F.Cu) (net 16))
 (via (at 184.404 113.284) (size 0.6) (drill 0.4) (layers F.Cu B.Cu) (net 16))
 (segment (start 184.404 115.316) (end 184.404 113.284) (width 0.25) (layer B.Cu) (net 16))
 (segment (start 181.694 118.026) (end 184.404 115.316) (width 0.25) (layer B.Cu) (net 16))
 (segment (start 182.118 112.252) (end 183.372 112.252) (width 0.25) (layer F.Cu) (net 17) (status 400000))
 (segment (start 183.642 98.298) (end 182.71 98.298) (width 0.25) (layer B.Cu) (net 17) (status 800000))
 (segment (start 184.404 99.06) (end 183.642 98.298) (width 0.25) (layer B.Cu) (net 17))
 (segment (start 184.404 112.268) (end 184.404 99.06) (width 0.25) (layer B.Cu) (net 17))
 (segment (start 184.15 112.522) (end 184.404 112.268) (width 0.25) (layer B.Cu) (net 17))
 (segment (start 183.642 112.522) (end 184.15 112.522) (width 0.25) (layer B.Cu) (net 17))
 (via (at 183.642 112.522) (size 0.6) (drill 0.4) (layers F.Cu B.Cu) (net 17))
 (segment (start 183.372 112.252) (end 183.642 112.522) (width 0.25) (layer F.Cu) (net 17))
 (segment (start 175.768 118.702) (end 177.546 118.702) (width 0.25) (layer B.Cu) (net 7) (status C00000))
 (segment (start 183.472 104.14) (end 183.472 107.696) (width 0.25) (layer B.Cu) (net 7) (status C00000))
 (segment (start 183.472 107.696) (end 183.472 111.252) (width 0.25) (layer B.Cu) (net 7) (status C00000))
 (segment (start 183.472 111.252) (end 183.472 111.676) (width 0.25) (layer B.Cu) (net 7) (status C00000))
 (segment (start 183.472 111.676) (end 182.88 112.268) (width 0.25) (layer B.Cu) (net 7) (status 400000))
 (segment (start 182.88 116.078) (end 180.086 118.872) (width 0.25) (layer B.Cu) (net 7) (status 800000))
 (segment (start 182.88 112.268) (end 182.88 116.078) (width 0.25) (layer B.Cu) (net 7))
 (segment (start 180.086 118.872) (end 179.494 118.872) (width 0.25) (layer B.Cu) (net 7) (status C00000))
 (segment (start 179.494 118.872) (end 180.086 118.872) (width 0.25) (layer B.Cu) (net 7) (status C00000))
 (segment (start 183.134 111.59) (end 183.472 111.252) (width 0.25) (layer B.Cu) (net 7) (status C00000))
 (segment (start 174.244 114.3) (end 173.736 114.3) (width 0.25) (layer B.Cu) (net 7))
 (segment (start 173.736 114.3) (end 172.72 115.316) (width 0.25) (layer B.Cu) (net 7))
 (segment (start 172.72 115.316) (end 172.72 117.856) (width 0.25) (layer B.Cu) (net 7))
 (segment (start 172.72 117.856) (end 173.566 118.702) (width 0.25) (layer B.Cu) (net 7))
 (segment (start 173.566 118.702) (end 177.546 118.702) (width 0.25) (layer B.Cu) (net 7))
 (segment (start 177.546 118.702) (end 177.716 118.872) (width 0.25) (layer B.Cu) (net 7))
 (segment (start 177.716 118.872) (end 179.494 118.872) (width 0.25) (layer B.Cu) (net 7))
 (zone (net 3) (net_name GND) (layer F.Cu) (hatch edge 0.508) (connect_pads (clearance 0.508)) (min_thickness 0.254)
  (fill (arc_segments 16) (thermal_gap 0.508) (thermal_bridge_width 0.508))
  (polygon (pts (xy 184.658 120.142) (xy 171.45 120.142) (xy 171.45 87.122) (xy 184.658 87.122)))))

